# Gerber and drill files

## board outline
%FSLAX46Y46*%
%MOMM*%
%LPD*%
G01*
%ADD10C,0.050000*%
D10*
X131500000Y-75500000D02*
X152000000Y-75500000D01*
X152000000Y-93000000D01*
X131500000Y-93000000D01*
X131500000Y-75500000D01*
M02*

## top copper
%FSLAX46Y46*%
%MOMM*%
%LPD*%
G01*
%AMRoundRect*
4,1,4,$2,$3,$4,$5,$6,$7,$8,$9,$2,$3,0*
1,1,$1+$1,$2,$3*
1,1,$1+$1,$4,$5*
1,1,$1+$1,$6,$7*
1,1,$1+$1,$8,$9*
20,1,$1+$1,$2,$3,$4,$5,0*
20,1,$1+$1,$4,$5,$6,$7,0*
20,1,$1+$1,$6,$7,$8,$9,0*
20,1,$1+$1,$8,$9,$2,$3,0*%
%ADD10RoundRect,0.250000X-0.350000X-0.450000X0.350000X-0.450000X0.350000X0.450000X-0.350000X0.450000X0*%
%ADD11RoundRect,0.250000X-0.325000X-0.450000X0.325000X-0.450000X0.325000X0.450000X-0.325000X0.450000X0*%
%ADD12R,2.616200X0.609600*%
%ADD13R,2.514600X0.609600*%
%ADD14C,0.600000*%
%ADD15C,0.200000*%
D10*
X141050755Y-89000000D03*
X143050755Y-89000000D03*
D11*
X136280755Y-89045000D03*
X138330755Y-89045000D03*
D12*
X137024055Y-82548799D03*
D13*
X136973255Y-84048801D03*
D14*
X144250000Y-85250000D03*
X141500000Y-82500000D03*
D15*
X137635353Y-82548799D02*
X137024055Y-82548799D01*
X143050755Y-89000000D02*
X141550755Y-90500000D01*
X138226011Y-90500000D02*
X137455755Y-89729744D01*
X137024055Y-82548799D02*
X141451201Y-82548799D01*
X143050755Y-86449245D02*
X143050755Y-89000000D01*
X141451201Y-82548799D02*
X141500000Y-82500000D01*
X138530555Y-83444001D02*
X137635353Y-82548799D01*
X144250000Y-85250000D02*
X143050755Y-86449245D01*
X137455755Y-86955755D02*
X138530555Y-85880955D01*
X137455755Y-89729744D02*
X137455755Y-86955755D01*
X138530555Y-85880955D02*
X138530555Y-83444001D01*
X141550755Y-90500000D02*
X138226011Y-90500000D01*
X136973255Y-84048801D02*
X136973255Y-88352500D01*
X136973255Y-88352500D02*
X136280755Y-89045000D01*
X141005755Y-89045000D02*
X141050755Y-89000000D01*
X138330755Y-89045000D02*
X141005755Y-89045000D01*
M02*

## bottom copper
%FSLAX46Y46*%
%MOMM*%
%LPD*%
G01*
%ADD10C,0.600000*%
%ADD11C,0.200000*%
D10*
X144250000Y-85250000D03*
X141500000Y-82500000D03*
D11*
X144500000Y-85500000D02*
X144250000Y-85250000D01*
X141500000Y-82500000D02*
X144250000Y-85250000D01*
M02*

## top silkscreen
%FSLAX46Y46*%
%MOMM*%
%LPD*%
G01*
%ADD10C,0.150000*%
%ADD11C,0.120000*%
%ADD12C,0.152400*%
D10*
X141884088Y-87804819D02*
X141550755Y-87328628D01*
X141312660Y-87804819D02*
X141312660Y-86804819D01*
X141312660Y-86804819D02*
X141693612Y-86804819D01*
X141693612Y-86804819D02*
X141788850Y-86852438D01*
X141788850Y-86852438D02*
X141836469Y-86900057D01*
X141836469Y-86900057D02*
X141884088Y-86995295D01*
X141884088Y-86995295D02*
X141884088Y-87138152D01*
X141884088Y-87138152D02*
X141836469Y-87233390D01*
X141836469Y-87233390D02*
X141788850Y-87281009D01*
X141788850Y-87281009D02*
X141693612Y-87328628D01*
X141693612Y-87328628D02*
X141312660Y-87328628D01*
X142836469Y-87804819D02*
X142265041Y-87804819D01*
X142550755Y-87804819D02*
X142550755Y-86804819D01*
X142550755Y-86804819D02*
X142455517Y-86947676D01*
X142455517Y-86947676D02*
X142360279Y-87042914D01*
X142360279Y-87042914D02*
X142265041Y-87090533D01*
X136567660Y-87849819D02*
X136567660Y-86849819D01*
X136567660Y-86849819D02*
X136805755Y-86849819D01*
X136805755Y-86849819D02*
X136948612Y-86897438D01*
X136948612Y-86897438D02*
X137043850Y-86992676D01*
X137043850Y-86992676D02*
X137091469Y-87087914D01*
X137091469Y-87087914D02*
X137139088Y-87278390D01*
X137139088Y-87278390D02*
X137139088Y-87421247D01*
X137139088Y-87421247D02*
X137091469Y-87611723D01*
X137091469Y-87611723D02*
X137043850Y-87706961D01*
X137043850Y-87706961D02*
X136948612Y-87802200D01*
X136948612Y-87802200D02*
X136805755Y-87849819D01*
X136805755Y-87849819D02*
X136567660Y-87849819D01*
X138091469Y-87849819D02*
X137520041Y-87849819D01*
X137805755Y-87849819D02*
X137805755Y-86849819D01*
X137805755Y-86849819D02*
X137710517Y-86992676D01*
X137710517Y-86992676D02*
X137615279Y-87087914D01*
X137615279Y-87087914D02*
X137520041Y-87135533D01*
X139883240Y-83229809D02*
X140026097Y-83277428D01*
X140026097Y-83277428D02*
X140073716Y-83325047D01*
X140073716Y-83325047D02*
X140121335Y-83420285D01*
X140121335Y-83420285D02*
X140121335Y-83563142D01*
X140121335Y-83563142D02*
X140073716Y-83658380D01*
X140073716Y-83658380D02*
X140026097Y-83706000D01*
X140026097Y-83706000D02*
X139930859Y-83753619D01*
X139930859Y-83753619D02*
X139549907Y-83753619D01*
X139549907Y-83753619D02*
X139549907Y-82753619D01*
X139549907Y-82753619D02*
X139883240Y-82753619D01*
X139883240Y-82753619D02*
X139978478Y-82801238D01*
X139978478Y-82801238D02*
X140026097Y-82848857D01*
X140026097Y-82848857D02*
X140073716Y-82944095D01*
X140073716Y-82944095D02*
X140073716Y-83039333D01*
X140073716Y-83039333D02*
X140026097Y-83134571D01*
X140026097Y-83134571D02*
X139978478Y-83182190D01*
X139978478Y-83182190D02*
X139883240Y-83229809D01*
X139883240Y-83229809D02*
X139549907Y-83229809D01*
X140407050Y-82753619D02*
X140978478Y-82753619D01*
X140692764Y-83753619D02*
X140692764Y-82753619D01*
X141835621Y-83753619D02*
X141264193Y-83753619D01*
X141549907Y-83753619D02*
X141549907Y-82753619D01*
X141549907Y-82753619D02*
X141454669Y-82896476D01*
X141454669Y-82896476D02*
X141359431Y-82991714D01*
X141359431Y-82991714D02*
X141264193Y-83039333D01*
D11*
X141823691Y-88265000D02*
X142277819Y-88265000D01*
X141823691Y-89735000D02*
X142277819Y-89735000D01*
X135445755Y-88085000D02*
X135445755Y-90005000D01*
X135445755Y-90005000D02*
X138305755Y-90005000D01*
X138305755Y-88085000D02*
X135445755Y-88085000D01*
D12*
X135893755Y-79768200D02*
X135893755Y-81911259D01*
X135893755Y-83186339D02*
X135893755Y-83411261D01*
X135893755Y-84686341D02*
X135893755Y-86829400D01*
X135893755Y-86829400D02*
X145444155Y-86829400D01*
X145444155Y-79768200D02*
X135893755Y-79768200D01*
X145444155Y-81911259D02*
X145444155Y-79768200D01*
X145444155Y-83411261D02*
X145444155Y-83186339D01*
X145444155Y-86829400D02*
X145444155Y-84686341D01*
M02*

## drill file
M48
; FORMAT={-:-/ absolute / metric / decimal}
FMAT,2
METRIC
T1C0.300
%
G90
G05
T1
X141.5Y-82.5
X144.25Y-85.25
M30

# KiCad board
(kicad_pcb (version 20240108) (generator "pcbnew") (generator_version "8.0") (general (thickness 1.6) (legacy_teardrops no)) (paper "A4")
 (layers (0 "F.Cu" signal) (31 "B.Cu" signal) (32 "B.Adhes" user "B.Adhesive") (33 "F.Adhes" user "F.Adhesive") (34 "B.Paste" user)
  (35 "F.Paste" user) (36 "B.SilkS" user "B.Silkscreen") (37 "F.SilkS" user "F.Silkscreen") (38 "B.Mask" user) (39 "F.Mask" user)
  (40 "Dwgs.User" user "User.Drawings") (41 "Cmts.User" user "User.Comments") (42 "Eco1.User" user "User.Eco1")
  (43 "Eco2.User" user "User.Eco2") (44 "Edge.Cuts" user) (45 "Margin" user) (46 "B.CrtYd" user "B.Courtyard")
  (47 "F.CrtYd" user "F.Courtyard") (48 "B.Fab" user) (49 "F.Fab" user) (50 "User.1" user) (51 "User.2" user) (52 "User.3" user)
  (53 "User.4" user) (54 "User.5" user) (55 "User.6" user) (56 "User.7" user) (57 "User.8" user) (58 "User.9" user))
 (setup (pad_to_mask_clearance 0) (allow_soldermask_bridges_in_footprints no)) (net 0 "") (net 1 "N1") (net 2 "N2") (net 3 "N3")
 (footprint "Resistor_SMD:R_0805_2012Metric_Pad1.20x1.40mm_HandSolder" (layer "F.Cu") (at 142.050755 89)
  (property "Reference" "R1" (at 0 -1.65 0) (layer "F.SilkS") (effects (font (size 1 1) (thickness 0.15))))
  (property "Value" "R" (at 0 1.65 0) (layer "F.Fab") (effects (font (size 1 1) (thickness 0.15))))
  (fp_line (start -0.227064 -0.735) (end 0.227064 -0.735) (stroke (width 0.12) (type solid)) (layer "F.SilkS"))
  (fp_line (start -0.227064 0.735) (end 0.227064 0.735) (stroke (width 0.12) (type solid)) (layer "F.SilkS"))
  (pad "1" smd roundrect (at -1 0) (size 1.2 1.4) (layers "F.Cu" "F.Paste" "F.Mask") (roundrect_rratio 0.208333) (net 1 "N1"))
  (pad "2" smd roundrect (at 1 0) (size 1.2 1.4) (layers "F.Cu" "F.Paste" "F.Mask") (roundrect_rratio 0.208333) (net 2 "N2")))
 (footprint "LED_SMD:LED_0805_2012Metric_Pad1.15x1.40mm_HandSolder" (layer "F.Cu") (at 137.305755 89.045)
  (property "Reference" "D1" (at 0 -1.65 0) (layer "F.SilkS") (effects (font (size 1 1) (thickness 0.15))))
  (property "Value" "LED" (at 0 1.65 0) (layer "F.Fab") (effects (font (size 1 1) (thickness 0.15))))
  (fp_line (start -1.86 -0.96) (end -1.86 0.96) (stroke (width 0.12) (type solid)) (layer "F.SilkS"))
  (fp_line (start -1.86 0.96) (end 1 0.96) (stroke (width 0.12) (type solid)) (layer "F.SilkS"))
  (fp_line (start 1 -0.96) (end -1.86 -0.96) (stroke (width 0.12) (type solid)) (layer "F.SilkS"))
  (pad "1" smd roundrect (at -1.025 0) (size 1.15 1.4) (layers "F.Cu" "F.Paste" "F.Mask") (roundrect_rratio 0.217391) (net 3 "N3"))
  (pad "2" smd roundrect (at 1.025 0) (size 1.15 1.4) (layers "F.Cu" "F.Paste" "F.Mask") (roundrect_rratio 0.217391) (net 1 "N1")))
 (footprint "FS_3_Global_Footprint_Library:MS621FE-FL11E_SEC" (layer "F.Cu") (at 140.668955 83.2988)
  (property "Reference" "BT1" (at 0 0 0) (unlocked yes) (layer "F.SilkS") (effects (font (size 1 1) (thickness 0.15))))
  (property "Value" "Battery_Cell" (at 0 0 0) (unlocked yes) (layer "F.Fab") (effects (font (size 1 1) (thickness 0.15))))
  (fp_line (start -4.7752 -3.5306) (end -4.7752 -1.387541) (stroke (width 0.1524) (type solid)) (layer "F.SilkS"))
  (fp_line (start -4.7752 -0.112461) (end -4.7752 0.112461) (stroke (width 0.1524) (type solid)) (layer "F.SilkS"))
  (fp_line (start -4.7752 1.387541) (end -4.7752 3.5306) (stroke (width 0.1524) (type solid)) (layer "F.SilkS"))
  (fp_line (start -4.7752 3.5306) (end 4.7752 3.5306) (stroke (width 0.1524) (type solid)) (layer "F.SilkS"))
  (fp_line (start 4.7752 -3.5306) (end -4.7752 -3.5306) (stroke (width 0.1524) (type solid)) (layer "F.SilkS"))
  (fp_line (start 4.7752 -1.387541) (end 4.7752 -3.5306) (stroke (width 0.1524) (type solid)) (layer "F.SilkS"))
  (fp_line (start 4.7752 0.112461) (end 4.7752 -0.112461) (stroke (width 0.1524) (type solid)) (layer "F.SilkS"))
  (fp_line (start 4.7752 3.5306) (end 4.7752 1.387541) (stroke (width 0.1524) (type solid)) (layer "F.SilkS"))
  (pad "1" smd rect (at -3.6449 -0.750001) (size 2.6162 0.6096) (layers "F.Cu" "F.Paste" "F.Mask") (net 2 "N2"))
  (pad "2" smd rect (at -3.6957 0.750001) (size 2.5146 0.6096) (layers "F.Cu" "F.Paste" "F.Mask") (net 3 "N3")))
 (gr_rect (start 131.5 75.5) (end 152 93) (stroke (width 0.05) (type default)) (fill none) (layer "Edge.Cuts"))
 (segment (start 137.635353 82.548799) (end 137.024055 82.548799) (width 0.2) (layer "F.Cu") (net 2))
 (segment (start 143.050755 89) (end 141.550755 90.5) (width 0.2) (layer "F.Cu") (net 2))
 (segment (start 138.226011 90.5) (end 137.455755 89.729744) (width 0.2) (layer "F.Cu") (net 2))
 (segment (start 137.024055 82.548799) (end 141.451201 82.548799) (width 0.2) (layer "F.Cu") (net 2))
 (segment (start 143.050755 86.449245) (end 143.050755 89) (width 0.2) (layer "F.Cu") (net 2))
 (segment (start 141.451201 82.548799) (end 141.5 82.5) (width 0.2) (layer "F.Cu") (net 2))
 (segment (start 138.530555 83.444001) (end 137.635353 82.548799) (width 0.2) (layer "F.Cu") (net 2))
 (segment (start 144.25 85.25) (end 143.050755 86.449245) (width 0.2) (layer "F.Cu") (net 2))
 (segment (start 137.455755 86.955755) (end 138.530555 85.880955) (width 0.2) (layer "F.Cu") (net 2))
 (segment (start 137.455755 89.729744) (end 137.455755 86.955755) (width 0.2) (layer "F.Cu") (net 2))
 (segment (start 138.530555 85.880955) (end 138.530555 83.444001) (width 0.2) (layer "F.Cu") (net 2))
 (segment (start 141.550755 90.5) (end 138.226011 90.5) (width 0.2) (layer "F.Cu") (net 2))
 (via (at 144.25 85.25) (size 0.6) (drill 0.3) (layers "F.Cu" "B.Cu") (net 2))
 (via (at 141.5 82.5) (size 0.6) (drill 0.3) (layers "F.Cu" "B.Cu") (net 2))
 (segment (start 144.5 85.5) (end 144.25 85.25) (width 0.2) (layer "B.Cu") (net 2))
 (segment (start 141.5 82.5) (end 144.25 85.25) (width 0.2) (layer "B.Cu") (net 2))
 (segment (start 136.973255 84.048801) (end 136.973255 88.3525) (width 0.2) (layer "F.Cu") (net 3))
 (segment (start 136.973255 88.3525) (end 136.280755 89.045) (width 0.2) (layer "F.Cu") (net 3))
 (segment (start 141.005755 89.045) (end 141.050755 89) (width 0.2) (layer "F.Cu") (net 1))
 (segment (start 138.330755 89.045) (end 141.005755 89.045) (width 0.2) (layer "F.Cu") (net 1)))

